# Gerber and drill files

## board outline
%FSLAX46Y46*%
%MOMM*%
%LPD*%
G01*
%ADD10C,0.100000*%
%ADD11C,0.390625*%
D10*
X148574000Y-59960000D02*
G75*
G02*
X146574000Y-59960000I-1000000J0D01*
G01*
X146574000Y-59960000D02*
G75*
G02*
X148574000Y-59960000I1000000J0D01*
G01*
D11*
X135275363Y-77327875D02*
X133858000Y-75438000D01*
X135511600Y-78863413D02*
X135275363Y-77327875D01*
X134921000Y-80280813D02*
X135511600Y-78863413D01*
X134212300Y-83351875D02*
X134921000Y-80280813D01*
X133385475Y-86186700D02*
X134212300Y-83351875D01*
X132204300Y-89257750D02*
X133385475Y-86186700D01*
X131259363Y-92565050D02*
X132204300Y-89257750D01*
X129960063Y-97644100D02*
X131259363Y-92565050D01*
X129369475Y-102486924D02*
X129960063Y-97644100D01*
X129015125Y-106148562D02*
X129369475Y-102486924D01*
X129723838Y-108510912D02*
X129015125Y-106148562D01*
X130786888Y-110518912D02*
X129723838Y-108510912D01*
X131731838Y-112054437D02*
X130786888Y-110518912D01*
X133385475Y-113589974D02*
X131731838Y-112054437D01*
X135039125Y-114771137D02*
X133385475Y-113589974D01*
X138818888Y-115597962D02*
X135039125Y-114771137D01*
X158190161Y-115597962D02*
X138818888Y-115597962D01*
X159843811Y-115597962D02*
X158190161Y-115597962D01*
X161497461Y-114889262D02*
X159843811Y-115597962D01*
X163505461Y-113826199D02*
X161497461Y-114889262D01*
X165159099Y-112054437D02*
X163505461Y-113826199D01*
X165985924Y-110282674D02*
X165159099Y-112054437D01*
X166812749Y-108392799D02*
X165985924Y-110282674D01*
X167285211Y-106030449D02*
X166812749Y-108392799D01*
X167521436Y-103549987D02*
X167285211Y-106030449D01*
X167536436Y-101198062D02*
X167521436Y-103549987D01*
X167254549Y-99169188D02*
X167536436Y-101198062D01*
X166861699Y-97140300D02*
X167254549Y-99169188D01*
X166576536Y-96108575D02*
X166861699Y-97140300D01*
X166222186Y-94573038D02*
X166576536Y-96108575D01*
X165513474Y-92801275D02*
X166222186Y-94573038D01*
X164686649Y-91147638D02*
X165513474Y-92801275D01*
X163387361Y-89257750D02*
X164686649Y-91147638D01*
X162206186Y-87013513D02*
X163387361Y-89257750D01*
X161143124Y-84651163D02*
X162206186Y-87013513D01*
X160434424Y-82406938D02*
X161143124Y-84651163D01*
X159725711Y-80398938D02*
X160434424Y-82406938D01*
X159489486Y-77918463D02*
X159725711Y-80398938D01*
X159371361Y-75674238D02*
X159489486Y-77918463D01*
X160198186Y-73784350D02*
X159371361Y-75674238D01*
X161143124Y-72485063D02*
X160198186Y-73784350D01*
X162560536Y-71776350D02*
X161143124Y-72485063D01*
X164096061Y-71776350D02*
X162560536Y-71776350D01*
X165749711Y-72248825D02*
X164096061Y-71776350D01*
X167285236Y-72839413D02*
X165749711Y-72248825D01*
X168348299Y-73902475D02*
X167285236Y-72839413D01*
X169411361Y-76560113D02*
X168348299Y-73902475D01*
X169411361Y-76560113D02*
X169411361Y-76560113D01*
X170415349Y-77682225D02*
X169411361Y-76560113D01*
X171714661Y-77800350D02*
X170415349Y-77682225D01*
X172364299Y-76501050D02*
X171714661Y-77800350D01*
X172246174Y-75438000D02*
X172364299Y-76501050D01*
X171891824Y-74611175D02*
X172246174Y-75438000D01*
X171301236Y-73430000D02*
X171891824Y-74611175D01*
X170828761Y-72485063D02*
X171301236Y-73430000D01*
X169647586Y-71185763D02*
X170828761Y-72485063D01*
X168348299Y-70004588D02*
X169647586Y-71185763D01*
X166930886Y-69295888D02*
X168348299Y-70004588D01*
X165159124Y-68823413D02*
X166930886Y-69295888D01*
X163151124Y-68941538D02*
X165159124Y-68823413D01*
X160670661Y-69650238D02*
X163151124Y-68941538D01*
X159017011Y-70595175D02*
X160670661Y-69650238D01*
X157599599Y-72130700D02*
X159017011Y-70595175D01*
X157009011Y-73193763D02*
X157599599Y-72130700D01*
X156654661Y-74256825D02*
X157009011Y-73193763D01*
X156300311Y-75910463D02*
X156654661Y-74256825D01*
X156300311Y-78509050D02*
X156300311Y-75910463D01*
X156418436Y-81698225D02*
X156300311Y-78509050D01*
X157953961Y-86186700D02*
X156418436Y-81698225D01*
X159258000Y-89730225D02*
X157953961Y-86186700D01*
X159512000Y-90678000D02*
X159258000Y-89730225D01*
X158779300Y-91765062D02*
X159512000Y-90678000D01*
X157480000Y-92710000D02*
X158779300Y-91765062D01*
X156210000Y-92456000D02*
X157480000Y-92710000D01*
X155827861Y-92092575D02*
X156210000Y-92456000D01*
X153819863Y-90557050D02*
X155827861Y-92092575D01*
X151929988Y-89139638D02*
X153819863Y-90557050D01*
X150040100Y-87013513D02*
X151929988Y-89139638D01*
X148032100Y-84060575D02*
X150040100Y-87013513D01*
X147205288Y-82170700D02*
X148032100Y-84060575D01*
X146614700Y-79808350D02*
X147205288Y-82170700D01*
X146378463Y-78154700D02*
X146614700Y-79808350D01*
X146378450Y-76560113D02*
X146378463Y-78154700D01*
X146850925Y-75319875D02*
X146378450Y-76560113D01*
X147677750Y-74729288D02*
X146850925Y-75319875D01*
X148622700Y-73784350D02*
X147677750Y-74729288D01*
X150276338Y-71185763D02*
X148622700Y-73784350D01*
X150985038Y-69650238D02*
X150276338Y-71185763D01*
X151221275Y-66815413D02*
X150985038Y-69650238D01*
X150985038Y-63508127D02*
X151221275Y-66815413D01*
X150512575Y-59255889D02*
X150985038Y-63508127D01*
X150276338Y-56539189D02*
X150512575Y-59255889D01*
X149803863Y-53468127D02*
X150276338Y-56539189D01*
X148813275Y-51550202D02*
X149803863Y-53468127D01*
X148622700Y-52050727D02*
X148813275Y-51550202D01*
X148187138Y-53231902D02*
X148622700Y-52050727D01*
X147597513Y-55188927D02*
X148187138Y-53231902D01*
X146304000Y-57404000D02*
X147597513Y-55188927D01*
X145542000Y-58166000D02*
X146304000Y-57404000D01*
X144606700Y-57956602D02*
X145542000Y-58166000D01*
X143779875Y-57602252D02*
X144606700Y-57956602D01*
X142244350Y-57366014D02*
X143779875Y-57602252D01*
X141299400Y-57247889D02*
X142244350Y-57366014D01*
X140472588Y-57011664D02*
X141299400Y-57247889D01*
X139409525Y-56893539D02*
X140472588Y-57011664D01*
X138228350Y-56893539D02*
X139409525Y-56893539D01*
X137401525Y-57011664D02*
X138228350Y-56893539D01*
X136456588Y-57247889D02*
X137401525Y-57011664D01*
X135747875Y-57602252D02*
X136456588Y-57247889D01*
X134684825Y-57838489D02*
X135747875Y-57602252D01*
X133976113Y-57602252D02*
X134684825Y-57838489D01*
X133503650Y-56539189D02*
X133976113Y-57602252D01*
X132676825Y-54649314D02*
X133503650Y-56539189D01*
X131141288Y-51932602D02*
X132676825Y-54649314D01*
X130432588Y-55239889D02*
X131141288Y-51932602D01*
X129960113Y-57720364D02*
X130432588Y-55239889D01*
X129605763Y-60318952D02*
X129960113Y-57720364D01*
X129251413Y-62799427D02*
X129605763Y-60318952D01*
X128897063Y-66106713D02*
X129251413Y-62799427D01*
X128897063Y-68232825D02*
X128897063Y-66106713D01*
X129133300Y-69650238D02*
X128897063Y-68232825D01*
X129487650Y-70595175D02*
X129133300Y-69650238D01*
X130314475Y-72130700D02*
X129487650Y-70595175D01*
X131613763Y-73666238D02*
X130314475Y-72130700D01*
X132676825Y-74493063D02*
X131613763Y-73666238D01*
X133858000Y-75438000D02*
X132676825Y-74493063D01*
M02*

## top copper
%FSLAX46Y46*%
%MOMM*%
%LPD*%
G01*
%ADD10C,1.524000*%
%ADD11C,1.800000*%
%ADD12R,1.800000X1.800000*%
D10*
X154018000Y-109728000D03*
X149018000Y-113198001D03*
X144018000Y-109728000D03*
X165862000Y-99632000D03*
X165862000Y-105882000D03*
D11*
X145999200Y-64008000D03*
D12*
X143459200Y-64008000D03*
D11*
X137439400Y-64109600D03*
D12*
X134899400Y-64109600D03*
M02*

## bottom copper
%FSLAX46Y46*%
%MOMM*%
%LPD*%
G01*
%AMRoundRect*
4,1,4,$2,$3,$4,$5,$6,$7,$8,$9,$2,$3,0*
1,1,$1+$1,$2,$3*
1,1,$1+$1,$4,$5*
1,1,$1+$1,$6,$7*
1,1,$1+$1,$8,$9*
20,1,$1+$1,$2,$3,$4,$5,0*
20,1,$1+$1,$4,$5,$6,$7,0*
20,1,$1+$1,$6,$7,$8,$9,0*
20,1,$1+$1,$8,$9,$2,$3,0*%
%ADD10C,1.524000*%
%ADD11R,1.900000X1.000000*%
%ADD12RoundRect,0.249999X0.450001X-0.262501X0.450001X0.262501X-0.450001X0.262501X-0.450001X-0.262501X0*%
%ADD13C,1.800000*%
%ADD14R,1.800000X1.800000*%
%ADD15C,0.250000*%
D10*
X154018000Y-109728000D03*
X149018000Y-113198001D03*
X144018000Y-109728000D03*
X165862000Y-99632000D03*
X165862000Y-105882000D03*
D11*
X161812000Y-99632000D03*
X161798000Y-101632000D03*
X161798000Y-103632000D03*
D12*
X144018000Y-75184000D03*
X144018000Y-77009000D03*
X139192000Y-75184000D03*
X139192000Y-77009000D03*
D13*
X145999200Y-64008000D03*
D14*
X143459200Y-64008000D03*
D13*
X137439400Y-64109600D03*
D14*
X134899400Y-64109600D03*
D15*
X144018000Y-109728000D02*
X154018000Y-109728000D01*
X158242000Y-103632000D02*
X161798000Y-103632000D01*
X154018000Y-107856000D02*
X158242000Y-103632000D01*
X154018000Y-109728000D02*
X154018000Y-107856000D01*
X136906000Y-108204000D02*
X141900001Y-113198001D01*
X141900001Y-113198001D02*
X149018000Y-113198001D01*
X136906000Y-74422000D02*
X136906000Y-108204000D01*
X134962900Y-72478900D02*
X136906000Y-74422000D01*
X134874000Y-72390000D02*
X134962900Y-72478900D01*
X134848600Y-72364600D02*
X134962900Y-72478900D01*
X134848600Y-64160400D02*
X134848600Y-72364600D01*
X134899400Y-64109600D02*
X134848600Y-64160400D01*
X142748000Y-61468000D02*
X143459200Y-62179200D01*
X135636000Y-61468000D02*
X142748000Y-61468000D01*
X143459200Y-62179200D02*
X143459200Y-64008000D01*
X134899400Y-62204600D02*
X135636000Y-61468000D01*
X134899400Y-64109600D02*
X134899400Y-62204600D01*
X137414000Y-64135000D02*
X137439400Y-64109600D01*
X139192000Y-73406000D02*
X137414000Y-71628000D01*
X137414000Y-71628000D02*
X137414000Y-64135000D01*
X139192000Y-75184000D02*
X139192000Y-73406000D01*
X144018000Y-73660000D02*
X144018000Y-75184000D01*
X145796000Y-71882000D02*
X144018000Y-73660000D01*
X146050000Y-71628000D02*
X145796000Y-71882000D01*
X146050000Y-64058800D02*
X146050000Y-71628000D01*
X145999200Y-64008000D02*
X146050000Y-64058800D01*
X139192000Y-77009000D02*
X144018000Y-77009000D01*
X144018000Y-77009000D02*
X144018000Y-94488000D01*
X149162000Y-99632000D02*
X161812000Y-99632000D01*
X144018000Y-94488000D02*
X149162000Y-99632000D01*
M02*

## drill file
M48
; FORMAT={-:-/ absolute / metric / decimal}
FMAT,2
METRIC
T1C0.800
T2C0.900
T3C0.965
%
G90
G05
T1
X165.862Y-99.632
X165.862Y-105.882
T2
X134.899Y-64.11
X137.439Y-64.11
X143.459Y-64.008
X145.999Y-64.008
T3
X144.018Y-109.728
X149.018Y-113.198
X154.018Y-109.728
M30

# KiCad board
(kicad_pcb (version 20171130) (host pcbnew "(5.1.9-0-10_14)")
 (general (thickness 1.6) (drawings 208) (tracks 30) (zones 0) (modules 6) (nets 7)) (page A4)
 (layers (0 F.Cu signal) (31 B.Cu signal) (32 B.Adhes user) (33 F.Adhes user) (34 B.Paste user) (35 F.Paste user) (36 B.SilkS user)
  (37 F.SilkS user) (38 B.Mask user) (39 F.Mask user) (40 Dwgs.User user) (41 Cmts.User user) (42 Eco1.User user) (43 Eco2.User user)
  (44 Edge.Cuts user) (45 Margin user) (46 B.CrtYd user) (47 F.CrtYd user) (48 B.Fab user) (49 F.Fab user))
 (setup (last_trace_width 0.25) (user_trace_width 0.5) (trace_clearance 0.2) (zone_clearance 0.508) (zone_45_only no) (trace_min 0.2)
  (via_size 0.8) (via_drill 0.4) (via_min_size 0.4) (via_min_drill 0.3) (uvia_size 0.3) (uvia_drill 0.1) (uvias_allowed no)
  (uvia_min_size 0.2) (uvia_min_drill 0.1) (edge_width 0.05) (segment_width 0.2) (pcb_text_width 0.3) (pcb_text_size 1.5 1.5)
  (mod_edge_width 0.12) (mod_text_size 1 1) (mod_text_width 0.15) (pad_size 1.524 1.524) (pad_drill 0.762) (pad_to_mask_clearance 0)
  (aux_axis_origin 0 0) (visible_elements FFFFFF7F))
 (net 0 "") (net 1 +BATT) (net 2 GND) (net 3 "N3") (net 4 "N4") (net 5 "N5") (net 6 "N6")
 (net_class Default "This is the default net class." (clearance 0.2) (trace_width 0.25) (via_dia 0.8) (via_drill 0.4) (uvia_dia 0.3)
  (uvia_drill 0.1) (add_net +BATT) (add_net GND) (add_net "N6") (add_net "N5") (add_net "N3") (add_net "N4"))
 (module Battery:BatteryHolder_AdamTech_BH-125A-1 (layer B.Cu) (at 144.018 109.728)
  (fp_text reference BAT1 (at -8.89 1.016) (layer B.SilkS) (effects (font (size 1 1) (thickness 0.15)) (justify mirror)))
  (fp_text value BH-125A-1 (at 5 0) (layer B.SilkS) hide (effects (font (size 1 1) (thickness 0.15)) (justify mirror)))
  (pad POS2 thru_hole circle (at 10 0) (size 1.524 1.524) (drill 0.9652) (layers *.Cu *.Mask) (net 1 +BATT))
  (pad NEG thru_hole circle (at 5 3.470001) (size 1.524 1.524) (drill 0.9652) (layers *.Cu *.Mask) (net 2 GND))
  (pad POS1 thru_hole circle (at 0 0) (size 1.524 1.524) (drill 0.9652) (layers *.Cu *.Mask) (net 1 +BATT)))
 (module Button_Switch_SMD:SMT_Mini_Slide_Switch (layer B.Cu) (at 163.576 102.757 270)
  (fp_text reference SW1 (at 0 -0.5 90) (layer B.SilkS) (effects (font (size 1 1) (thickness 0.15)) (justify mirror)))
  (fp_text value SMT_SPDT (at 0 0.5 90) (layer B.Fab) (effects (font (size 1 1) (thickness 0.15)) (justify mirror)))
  (pad "" thru_hole circle (at -3.125 -2.286 270) (size 1.524 1.524) (drill 0.8) (layers *.Cu *.Mask))
  (pad "" thru_hole circle (at 3.125 -2.286 270) (size 1.524 1.524) (drill 0.8) (layers *.Cu *.Mask))
  (pad 1 smd rect (at -3.125 1.764 270) (size 1 1.9) (layers B.Cu B.Paste B.Mask) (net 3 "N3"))
  (pad 2 smd rect (at -1.125 1.778 270) (size 1 1.9) (layers B.Cu B.Paste B.Mask) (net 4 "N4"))
  (pad 3 smd rect (at 0.875 1.778 270) (size 1 1.9) (layers B.Cu B.Paste B.Mask) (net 1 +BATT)))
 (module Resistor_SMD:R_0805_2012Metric (layer B.Cu) (at 144.018 76.0965 90)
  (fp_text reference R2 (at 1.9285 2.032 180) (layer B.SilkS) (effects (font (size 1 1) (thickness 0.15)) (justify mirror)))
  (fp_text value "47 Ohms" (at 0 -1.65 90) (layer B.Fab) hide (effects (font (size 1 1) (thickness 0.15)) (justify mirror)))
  (pad 2 smd roundrect (at 0.9125 0 90) (size 1.025 1.4) (layers B.Cu B.Paste B.Mask) (roundrect_rratio 0.2439014634146341) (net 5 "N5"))
  (pad 1 smd roundrect (at -0.9125 0 90) (size 1.025 1.4) (layers B.Cu B.Paste B.Mask) (roundrect_rratio 0.2439014634146341) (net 3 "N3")))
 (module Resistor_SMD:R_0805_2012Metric (layer B.Cu) (at 139.192 76.0965 90)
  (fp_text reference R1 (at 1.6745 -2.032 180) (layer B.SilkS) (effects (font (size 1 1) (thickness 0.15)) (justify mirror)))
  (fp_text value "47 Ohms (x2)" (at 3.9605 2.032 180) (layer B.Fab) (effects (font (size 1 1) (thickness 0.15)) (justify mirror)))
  (pad 2 smd roundrect (at 0.9125 0 90) (size 1.025 1.4) (layers B.Cu B.Paste B.Mask) (roundrect_rratio 0.2439014634146341) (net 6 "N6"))
  (pad 1 smd roundrect (at -0.9125 0 90) (size 1.025 1.4) (layers B.Cu B.Paste B.Mask) (roundrect_rratio 0.2439014634146341) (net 3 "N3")))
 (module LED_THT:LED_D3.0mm (layer B.Cu) (at 143.4592 64.008)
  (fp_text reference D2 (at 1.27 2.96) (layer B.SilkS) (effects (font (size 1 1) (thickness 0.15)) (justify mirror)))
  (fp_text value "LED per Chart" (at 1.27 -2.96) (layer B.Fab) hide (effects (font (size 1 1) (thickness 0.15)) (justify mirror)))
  (pad 2 thru_hole circle (at 2.54 0) (size 1.8 1.8) (drill 0.9) (layers *.Cu *.Mask) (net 5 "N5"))
  (pad 1 thru_hole rect (at 0 0) (size 1.8 1.8) (drill 0.9) (layers *.Cu *.Mask) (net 2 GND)))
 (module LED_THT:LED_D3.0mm (layer B.Cu) (at 134.8994 64.1096)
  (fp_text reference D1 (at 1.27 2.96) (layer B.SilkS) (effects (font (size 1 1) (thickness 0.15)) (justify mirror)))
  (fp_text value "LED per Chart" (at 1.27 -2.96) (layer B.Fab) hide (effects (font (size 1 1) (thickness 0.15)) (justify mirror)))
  (pad 2 thru_hole circle (at 2.54 0) (size 1.8 1.8) (drill 0.9) (layers *.Cu *.Mask) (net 6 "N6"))
  (pad 1 thru_hole rect (at 0 0) (size 1.8 1.8) (drill 0.9) (layers *.Cu *.Mask) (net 2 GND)))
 (gr_circle (center 147.574 59.96) (end 148.574 59.96) (layer Edge.Cuts) (width 0.1))
 (gr_line (start 135.275363 77.327875) (end 133.858 75.438) (layer Edge.Cuts) (width 0.390625))
 (gr_line (start 135.5116 78.863413) (end 135.275363 77.327875) (layer Edge.Cuts) (width 0.390625))
 (gr_line (start 134.921 80.280813) (end 135.5116 78.863413) (layer Edge.Cuts) (width 0.390625))
 (gr_line (start 134.2123 83.351875) (end 134.921 80.280813) (layer Edge.Cuts) (width 0.390625))
 (gr_line (start 133.385475 86.1867) (end 134.2123 83.351875) (layer Edge.Cuts) (width 0.390625))
 (gr_line (start 132.2043 89.25775) (end 133.385475 86.1867) (layer Edge.Cuts) (width 0.390625))
 (gr_line (start 131.259363 92.56505) (end 132.2043 89.25775) (layer Edge.Cuts) (width 0.390625))
 (gr_line (start 129.960063 97.6441) (end 131.259363 92.56505) (layer Edge.Cuts) (width 0.390625))
 (gr_line (start 129.369475 102.486924) (end 129.960063 97.6441) (layer Edge.Cuts) (width 0.390625))
 (gr_line (start 129.015125 106.148562) (end 129.369475 102.486924) (layer Edge.Cuts) (width 0.390625))
 (gr_line (start 129.723838 108.510912) (end 129.015125 106.148562) (layer Edge.Cuts) (width 0.390625))
 (gr_line (start 130.786888 110.518912) (end 129.723838 108.510912) (layer Edge.Cuts) (width 0.390625))
 (gr_line (start 131.731838 112.054437) (end 130.786888 110.518912) (layer Edge.Cuts) (width 0.390625))
 (gr_line (start 133.385475 113.589974) (end 131.731838 112.054437) (layer Edge.Cuts) (width 0.390625))
 (gr_line (start 135.039125 114.771137) (end 133.385475 113.589974) (layer Edge.Cuts) (width 0.390625))
 (gr_line (start 138.818888 115.597962) (end 135.039125 114.771137) (layer Edge.Cuts) (width 0.390625))
 (gr_line (start 158.190161 115.597962) (end 138.818888 115.597962) (layer Edge.Cuts) (width 0.390625))
 (gr_line (start 159.843811 115.597962) (end 158.190161 115.597962) (layer Edge.Cuts) (width 0.390625))
 (gr_line (start 161.497461 114.889262) (end 159.843811 115.597962) (layer Edge.Cuts) (width 0.390625))
 (gr_line (start 163.505461 113.826199) (end 161.497461 114.889262) (layer Edge.Cuts) (width 0.390625))
 (gr_line (start 165.159099 112.054437) (end 163.505461 113.826199) (layer Edge.Cuts) (width 0.390625))
 (gr_line (start 165.985924 110.282674) (end 165.159099 112.054437) (layer Edge.Cuts) (width 0.390625))
 (gr_line (start 166.812749 108.392799) (end 165.985924 110.282674) (layer Edge.Cuts) (width 0.390625))
 (gr_line (start 167.285211 106.030449) (end 166.812749 108.392799) (layer Edge.Cuts) (width 0.390625))
 (gr_line (start 167.521436 103.549987) (end 167.285211 106.030449) (layer Edge.Cuts) (width 0.390625))
 (gr_line (start 167.536436 101.198062) (end 167.521436 103.549987) (layer Edge.Cuts) (width 0.390625))
 (gr_line (start 167.254549 99.169188) (end 167.536436 101.198062) (layer Edge.Cuts) (width 0.390625))
 (gr_line (start 166.861699 97.1403) (end 167.254549 99.169188) (layer Edge.Cuts) (width 0.390625))
 (gr_line (start 166.576536 96.108575) (end 166.861699 97.1403) (layer Edge.Cuts) (width 0.390625))
 (gr_line (start 166.222186 94.573038) (end 166.576536 96.108575) (layer Edge.Cuts) (width 0.390625))
 (gr_line (start 165.513474 92.801275) (end 166.222186 94.573038) (layer Edge.Cuts) (width 0.390625))
 (gr_line (start 164.686649 91.147638) (end 165.513474 92.801275) (layer Edge.Cuts) (width 0.390625))
 (gr_line (start 163.387361 89.25775) (end 164.686649 91.147638) (layer Edge.Cuts) (width 0.390625))
 (gr_line (start 162.206186 87.013513) (end 163.387361 89.25775) (layer Edge.Cuts) (width 0.390625))
 (gr_line (start 161.143124 84.651163) (end 162.206186 87.013513) (layer Edge.Cuts) (width 0.390625))
 (gr_line (start 160.434424 82.406938) (end 161.143124 84.651163) (layer Edge.Cuts) (width 0.390625))
 (gr_line (start 159.725711 80.398938) (end 160.434424 82.406938) (layer Edge.Cuts) (width 0.390625))
 (gr_line (start 159.489486 77.918463) (end 159.725711 80.398938) (layer Edge.Cuts) (width 0.390625))
 (gr_line (start 159.371361 75.674238) (end 159.489486 77.918463) (layer Edge.Cuts) (width 0.390625))
 (gr_line (start 160.198186 73.78435) (end 159.371361 75.674238) (layer Edge.Cuts) (width 0.390625))
 (gr_line (start 161.143124 72.485063) (end 160.198186 73.78435) (layer Edge.Cuts) (width 0.390625))
 (gr_line (start 162.560536 71.77635) (end 161.143124 72.485063) (layer Edge.Cuts) (width 0.390625))
 (gr_line (start 164.096061 71.77635) (end 162.560536 71.77635) (layer Edge.Cuts) (width 0.390625))
 (gr_line (start 165.749711 72.248825) (end 164.096061 71.77635) (layer Edge.Cuts) (width 0.390625))
 (gr_line (start 167.285236 72.839413) (end 165.749711 72.248825) (layer Edge.Cuts) (width 0.390625))
 (gr_line (start 168.348299 73.902475) (end 167.285236 72.839413) (layer Edge.Cuts) (width 0.390625))
 (gr_line (start 169.411361 76.560113) (end 168.348299 73.902475) (layer Edge.Cuts) (width 0.390625))
 (gr_line (start 169.411361 76.560113) (end 169.411361 76.560113) (layer Edge.Cuts) (width 0.390625))
 (gr_line (start 170.415349 77.682225) (end 169.411361 76.560113) (layer Edge.Cuts) (width 0.390625))
 (gr_line (start 171.714661 77.80035) (end 170.415349 77.682225) (layer Edge.Cuts) (width 0.390625))
 (gr_line (start 172.364299 76.50105) (end 171.714661 77.80035) (layer Edge.Cuts) (width 0.390625))
 (gr_line (start 172.246174 75.438) (end 172.364299 76.50105) (layer Edge.Cuts) (width 0.390625))
 (gr_line (start 171.891824 74.611175) (end 172.246174 75.438) (layer Edge.Cuts) (width 0.390625))
 (gr_line (start 171.301236 73.43) (end 171.891824 74.611175) (layer Edge.Cuts) (width 0.390625))
 (gr_line (start 170.828761 72.485063) (end 171.301236 73.43) (layer Edge.Cuts) (width 0.390625))
 (gr_line (start 169.647586 71.185763) (end 170.828761 72.485063) (layer Edge.Cuts) (width 0.390625))
 (gr_line (start 168.348299 70.004588) (end 169.647586 71.185763) (layer Edge.Cuts) (width 0.390625))
 (gr_line (start 166.930886 69.295888) (end 168.348299 70.004588) (layer Edge.Cuts) (width 0.390625))
 (gr_line (start 165.159124 68.823413) (end 166.930886 69.295888) (layer Edge.Cuts) (width 0.390625))
 (gr_line (start 163.151124 68.941538) (end 165.159124 68.823413) (layer Edge.Cuts) (width 0.390625))
 (gr_line (start 160.670661 69.650238) (end 163.151124 68.941538) (layer Edge.Cuts) (width 0.390625))
 (gr_line (start 159.017011 70.595175) (end 160.670661 69.650238) (layer Edge.Cuts) (width 0.390625))
 (gr_line (start 157.599599 72.1307) (end 159.017011 70.595175) (layer Edge.Cuts) (width 0.390625))
 (gr_line (start 157.009011 73.193763) (end 157.599599 72.1307) (layer Edge.Cuts) (width 0.390625))
 (gr_line (start 156.654661 74.256825) (end 157.009011 73.193763) (layer Edge.Cuts) (width 0.390625))
 (gr_line (start 156.300311 75.910463) (end 156.654661 74.256825) (layer Edge.Cuts) (width 0.390625))
 (gr_line (start 156.300311 78.50905) (end 156.300311 75.910463) (layer Edge.Cuts) (width 0.390625))
 (gr_line (start 156.418436 81.698225) (end 156.300311 78.50905) (layer Edge.Cuts) (width 0.390625))
 (gr_line (start 157.953961 86.1867) (end 156.418436 81.698225) (layer Edge.Cuts) (width 0.390625))
 (gr_line (start 159.258 89.730225) (end 157.953961 86.1867) (layer Edge.Cuts) (width 0.390625))
 (gr_line (start 159.512 90.678) (end 159.258 89.730225) (layer Edge.Cuts) (width 0.390625))
 (gr_line (start 158.7793 91.765062) (end 159.512 90.678) (layer Edge.Cuts) (width 0.390625))
 (gr_line (start 157.48 92.71) (end 158.7793 91.765062) (layer Edge.Cuts) (width 0.390625))
 (gr_line (start 156.21 92.456) (end 157.48 92.71) (layer Edge.Cuts) (width 0.390625))
 (gr_line (start 155.827861 92.092575) (end 156.21 92.456) (layer Edge.Cuts) (width 0.390625))
 (gr_line (start 153.819863 90.55705) (end 155.827861 92.092575) (layer Edge.Cuts) (width 0.390625))
 (gr_line (start 151.929988 89.139638) (end 153.819863 90.55705) (layer Edge.Cuts) (width 0.390625))
 (gr_line (start 150.0401 87.013513) (end 151.929988 89.139638) (layer Edge.Cuts) (width 0.390625))
 (gr_line (start 148.0321 84.060575) (end 150.0401 87.013513) (layer Edge.Cuts) (width 0.390625))
 (gr_line (start 147.205288 82.1707) (end 148.0321 84.060575) (layer Edge.Cuts) (width 0.390625))
 (gr_line (start 146.6147 79.80835) (end 147.205288 82.1707) (layer Edge.Cuts) (width 0.390625))
 (gr_line (start 146.378463 78.1547) (end 146.6147 79.80835) (layer Edge.Cuts) (width 0.390625))
 (gr_line (start 146.37845 76.560113) (end 146.378463 78.1547) (layer Edge.Cuts) (width 0.390625))
 (gr_line (start 146.850925 75.319875) (end 146.37845 76.560113) (layer Edge.Cuts) (width 0.390625))
 (gr_line (start 147.67775 74.729288) (end 146.850925 75.319875) (layer Edge.Cuts) (width 0.390625))
 (gr_line (start 148.6227 73.78435) (end 147.67775 74.729288) (layer Edge.Cuts) (width 0.390625))
 (gr_line (start 150.276338 71.185763) (end 148.6227 73.78435) (layer Edge.Cuts) (width 0.390625))
 (gr_line (start 150.985038 69.650238) (end 150.276338 71.185763) (layer Edge.Cuts) (width 0.390625))
 (gr_line (start 151.221275 66.815413) (end 150.985038 69.650238) (layer Edge.Cuts) (width 0.390625))
 (gr_line (start 150.985038 63.508127) (end 151.221275 66.815413) (layer Edge.Cuts) (width 0.390625))
 (gr_line (start 150.512575 59.255889) (end 150.985038 63.508127) (layer Edge.Cuts) (width 0.390625))
 (gr_line (start 150.276338 56.539189) (end 150.512575 59.255889) (layer Edge.Cuts) (width 0.390625))
 (gr_line (start 149.803863 53.468127) (end 150.276338 56.539189) (layer Edge.Cuts) (width 0.390625))
 (gr_line (start 148.813275 51.550202) (end 149.803863 53.468127) (layer Edge.Cuts) (width 0.390625))
 (gr_line (start 148.6227 52.050727) (end 148.813275 51.550202) (layer Edge.Cuts) (width 0.390625))
 (gr_line (start 148.187138 53.231902) (end 148.6227 52.050727) (layer Edge.Cuts) (width 0.390625))
 (gr_line (start 147.597513 55.188927) (end 148.187138 53.231902) (layer Edge.Cuts) (width 0.390625))
 (gr_line (start 146.304 57.404) (end 147.597513 55.188927) (layer Edge.Cuts) (width 0.390625))
 (gr_line (start 145.542 58.166) (end 146.304 57.404) (layer Edge.Cuts) (width 0.390625))
 (gr_line (start 144.6067 57.956602) (end 145.542 58.166) (layer Edge.Cuts) (width 0.390625))
 (gr_line (start 143.779875 57.602252) (end 144.6067 57.956602) (layer Edge.Cuts) (width 0.390625))
 (gr_line (start 142.24435 57.366014) (end 143.779875 57.602252) (layer Edge.Cuts) (width 0.390625))
 (gr_line (start 141.2994 57.247889) (end 142.24435 57.366014) (layer Edge.Cuts) (width 0.390625))
 (gr_line (start 140.472588 57.011664) (end 141.2994 57.247889) (layer Edge.Cuts) (width 0.390625))
 (gr_line (start 139.409525 56.893539) (end 140.472588 57.011664) (layer Edge.Cuts) (width 0.390625))
 (gr_line (start 138.22835 56.893539) (end 139.409525 56.893539) (layer Edge.Cuts) (width 0.390625))
 (gr_line (start 137.401525 57.011664) (end 138.22835 56.893539) (layer Edge.Cuts) (width 0.390625))
 (gr_line (start 136.456588 57.247889) (end 137.401525 57.011664) (layer Edge.Cuts) (width 0.390625))
 (gr_line (start 135.747875 57.602252) (end 136.456588 57.247889) (layer Edge.Cuts) (width 0.390625))
 (gr_line (start 134.684825 57.838489) (end 135.747875 57.602252) (layer Edge.Cuts) (width 0.390625))
 (gr_line (start 133.976113 57.602252) (end 134.684825 57.838489) (layer Edge.Cuts) (width 0.390625))
 (gr_line (start 133.50365 56.539189) (end 133.976113 57.602252) (layer Edge.Cuts) (width 0.390625))
 (gr_line (start 132.676825 54.649314) (end 133.50365 56.539189) (layer Edge.Cuts) (width 0.390625))
 (gr_line (start 131.141288 51.932602) (end 132.676825 54.649314) (layer Edge.Cuts) (width 0.390625))
 (gr_line (start 130.432588 55.239889) (end 131.141288 51.932602) (layer Edge.Cuts) (width 0.390625))
 (gr_line (start 129.960113 57.720364) (end 130.432588 55.239889) (layer Edge.Cuts) (width 0.390625))
 (gr_line (start 129.605763 60.318952) (end 129.960113 57.720364) (layer Edge.Cuts) (width 0.390625))
 (gr_line (start 129.251413 62.799427) (end 129.605763 60.318952) (layer Edge.Cuts) (width 0.390625))
 (gr_line (start 128.897063 66.106713) (end 129.251413 62.799427) (layer Edge.Cuts) (width 0.390625))
 (gr_line (start 128.897063 68.232825) (end 128.897063 66.106713) (layer Edge.Cuts) (width 0.390625))
 (gr_line (start 129.1333 69.650238) (end 128.897063 68.232825) (layer Edge.Cuts) (width 0.390625))
 (gr_line (start 129.48765 70.595175) (end 129.1333 69.650238) (layer Edge.Cuts) (width 0.390625))
 (gr_line (start 130.314475 72.1307) (end 129.48765 70.595175) (layer Edge.Cuts) (width 0.390625))
 (gr_line (start 131.613763 73.666238) (end 130.314475 72.1307) (layer Edge.Cuts) (width 0.390625))
 (gr_line (start 132.676825 74.493063) (end 131.613763 73.666238) (layer Edge.Cuts) (width 0.390625))
 (gr_line (start 133.858 75.438) (end 132.676825 74.493063) (layer Edge.Cuts) (width 0.390625))
 (segment (start 144.018 109.728) (end 154.018 109.728) (width 0.25) (layer B.Cu) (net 1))
 (segment (start 158.242 103.632) (end 161.798 103.632) (width 0.25) (layer B.Cu) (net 1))
 (segment (start 154.018 107.856) (end 158.242 103.632) (width 0.25) (layer B.Cu) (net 1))
 (segment (start 154.018 109.728) (end 154.018 107.856) (width 0.25) (layer B.Cu) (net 1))
 (segment (start 136.906 108.204) (end 141.900001 113.198001) (width 0.25) (layer B.Cu) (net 2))
 (segment (start 141.900001 113.198001) (end 149.018 113.198001) (width 0.25) (layer B.Cu) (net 2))
 (segment (start 136.906 74.422) (end 136.906 108.204) (width 0.25) (layer B.Cu) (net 2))
 (segment (start 134.9629 72.4789) (end 136.906 74.422) (width 0.25) (layer B.Cu) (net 2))
 (segment (start 134.874 72.39) (end 134.9629 72.4789) (width 0.25) (layer B.Cu) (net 2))
 (segment (start 134.8486 72.3646) (end 134.9629 72.4789) (width 0.25) (layer B.Cu) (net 2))
 (segment (start 134.8486 64.1604) (end 134.8486 72.3646) (width 0.25) (layer B.Cu) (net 2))
 (segment (start 134.8994 64.1096) (end 134.8486 64.1604) (width 0.25) (layer B.Cu) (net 2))
 (segment (start 142.748 61.468) (end 143.4592 62.1792) (width 0.25) (layer B.Cu) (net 2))
 (segment (start 135.636 61.468) (end 142.748 61.468) (width 0.25) (layer B.Cu) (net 2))
 (segment (start 143.4592 62.1792) (end 143.4592 64.008) (width 0.25) (layer B.Cu) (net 2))
 (segment (start 134.8994 62.2046) (end 135.636 61.468) (width 0.25) (layer B.Cu) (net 2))
 (segment (start 134.8994 64.1096) (end 134.8994 62.2046) (width 0.25) (layer B.Cu) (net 2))
 (segment (start 137.414 64.135) (end 137.4394 64.1096) (width 0.25) (layer B.Cu) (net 6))
 (segment (start 139.192 73.406) (end 137.414 71.628) (width 0.25) (layer B.Cu) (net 6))
 (segment (start 137.414 71.628) (end 137.414 64.135) (width 0.25) (layer B.Cu) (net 6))
 (segment (start 139.192 75.184) (end 139.192 73.406) (width 0.25) (layer B.Cu) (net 6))
 (segment (start 144.018 73.66) (end 144.018 75.184) (width 0.25) (layer B.Cu) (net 5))
 (segment (start 145.796 71.882) (end 144.018 73.66) (width 0.25) (layer B.Cu) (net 5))
 (segment (start 146.05 71.628) (end 145.796 71.882) (width 0.25) (layer B.Cu) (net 5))
 (segment (start 146.05 64.0588) (end 146.05 71.628) (width 0.25) (layer B.Cu) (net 5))
 (segment (start 145.9992 64.008) (end 146.05 64.0588) (width 0.25) (layer B.Cu) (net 5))
 (segment (start 139.192 77.009) (end 144.018 77.009) (width 0.25) (layer B.Cu) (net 3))
 (segment (start 144.018 77.009) (end 144.018 94.488) (width 0.25) (layer B.Cu) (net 3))
 (segment (start 149.162 99.632) (end 161.812 99.632) (width 0.25) (layer B.Cu) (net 3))
 (segment (start 144.018 94.488) (end 149.162 99.632) (width 0.25) (layer B.Cu) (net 3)))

